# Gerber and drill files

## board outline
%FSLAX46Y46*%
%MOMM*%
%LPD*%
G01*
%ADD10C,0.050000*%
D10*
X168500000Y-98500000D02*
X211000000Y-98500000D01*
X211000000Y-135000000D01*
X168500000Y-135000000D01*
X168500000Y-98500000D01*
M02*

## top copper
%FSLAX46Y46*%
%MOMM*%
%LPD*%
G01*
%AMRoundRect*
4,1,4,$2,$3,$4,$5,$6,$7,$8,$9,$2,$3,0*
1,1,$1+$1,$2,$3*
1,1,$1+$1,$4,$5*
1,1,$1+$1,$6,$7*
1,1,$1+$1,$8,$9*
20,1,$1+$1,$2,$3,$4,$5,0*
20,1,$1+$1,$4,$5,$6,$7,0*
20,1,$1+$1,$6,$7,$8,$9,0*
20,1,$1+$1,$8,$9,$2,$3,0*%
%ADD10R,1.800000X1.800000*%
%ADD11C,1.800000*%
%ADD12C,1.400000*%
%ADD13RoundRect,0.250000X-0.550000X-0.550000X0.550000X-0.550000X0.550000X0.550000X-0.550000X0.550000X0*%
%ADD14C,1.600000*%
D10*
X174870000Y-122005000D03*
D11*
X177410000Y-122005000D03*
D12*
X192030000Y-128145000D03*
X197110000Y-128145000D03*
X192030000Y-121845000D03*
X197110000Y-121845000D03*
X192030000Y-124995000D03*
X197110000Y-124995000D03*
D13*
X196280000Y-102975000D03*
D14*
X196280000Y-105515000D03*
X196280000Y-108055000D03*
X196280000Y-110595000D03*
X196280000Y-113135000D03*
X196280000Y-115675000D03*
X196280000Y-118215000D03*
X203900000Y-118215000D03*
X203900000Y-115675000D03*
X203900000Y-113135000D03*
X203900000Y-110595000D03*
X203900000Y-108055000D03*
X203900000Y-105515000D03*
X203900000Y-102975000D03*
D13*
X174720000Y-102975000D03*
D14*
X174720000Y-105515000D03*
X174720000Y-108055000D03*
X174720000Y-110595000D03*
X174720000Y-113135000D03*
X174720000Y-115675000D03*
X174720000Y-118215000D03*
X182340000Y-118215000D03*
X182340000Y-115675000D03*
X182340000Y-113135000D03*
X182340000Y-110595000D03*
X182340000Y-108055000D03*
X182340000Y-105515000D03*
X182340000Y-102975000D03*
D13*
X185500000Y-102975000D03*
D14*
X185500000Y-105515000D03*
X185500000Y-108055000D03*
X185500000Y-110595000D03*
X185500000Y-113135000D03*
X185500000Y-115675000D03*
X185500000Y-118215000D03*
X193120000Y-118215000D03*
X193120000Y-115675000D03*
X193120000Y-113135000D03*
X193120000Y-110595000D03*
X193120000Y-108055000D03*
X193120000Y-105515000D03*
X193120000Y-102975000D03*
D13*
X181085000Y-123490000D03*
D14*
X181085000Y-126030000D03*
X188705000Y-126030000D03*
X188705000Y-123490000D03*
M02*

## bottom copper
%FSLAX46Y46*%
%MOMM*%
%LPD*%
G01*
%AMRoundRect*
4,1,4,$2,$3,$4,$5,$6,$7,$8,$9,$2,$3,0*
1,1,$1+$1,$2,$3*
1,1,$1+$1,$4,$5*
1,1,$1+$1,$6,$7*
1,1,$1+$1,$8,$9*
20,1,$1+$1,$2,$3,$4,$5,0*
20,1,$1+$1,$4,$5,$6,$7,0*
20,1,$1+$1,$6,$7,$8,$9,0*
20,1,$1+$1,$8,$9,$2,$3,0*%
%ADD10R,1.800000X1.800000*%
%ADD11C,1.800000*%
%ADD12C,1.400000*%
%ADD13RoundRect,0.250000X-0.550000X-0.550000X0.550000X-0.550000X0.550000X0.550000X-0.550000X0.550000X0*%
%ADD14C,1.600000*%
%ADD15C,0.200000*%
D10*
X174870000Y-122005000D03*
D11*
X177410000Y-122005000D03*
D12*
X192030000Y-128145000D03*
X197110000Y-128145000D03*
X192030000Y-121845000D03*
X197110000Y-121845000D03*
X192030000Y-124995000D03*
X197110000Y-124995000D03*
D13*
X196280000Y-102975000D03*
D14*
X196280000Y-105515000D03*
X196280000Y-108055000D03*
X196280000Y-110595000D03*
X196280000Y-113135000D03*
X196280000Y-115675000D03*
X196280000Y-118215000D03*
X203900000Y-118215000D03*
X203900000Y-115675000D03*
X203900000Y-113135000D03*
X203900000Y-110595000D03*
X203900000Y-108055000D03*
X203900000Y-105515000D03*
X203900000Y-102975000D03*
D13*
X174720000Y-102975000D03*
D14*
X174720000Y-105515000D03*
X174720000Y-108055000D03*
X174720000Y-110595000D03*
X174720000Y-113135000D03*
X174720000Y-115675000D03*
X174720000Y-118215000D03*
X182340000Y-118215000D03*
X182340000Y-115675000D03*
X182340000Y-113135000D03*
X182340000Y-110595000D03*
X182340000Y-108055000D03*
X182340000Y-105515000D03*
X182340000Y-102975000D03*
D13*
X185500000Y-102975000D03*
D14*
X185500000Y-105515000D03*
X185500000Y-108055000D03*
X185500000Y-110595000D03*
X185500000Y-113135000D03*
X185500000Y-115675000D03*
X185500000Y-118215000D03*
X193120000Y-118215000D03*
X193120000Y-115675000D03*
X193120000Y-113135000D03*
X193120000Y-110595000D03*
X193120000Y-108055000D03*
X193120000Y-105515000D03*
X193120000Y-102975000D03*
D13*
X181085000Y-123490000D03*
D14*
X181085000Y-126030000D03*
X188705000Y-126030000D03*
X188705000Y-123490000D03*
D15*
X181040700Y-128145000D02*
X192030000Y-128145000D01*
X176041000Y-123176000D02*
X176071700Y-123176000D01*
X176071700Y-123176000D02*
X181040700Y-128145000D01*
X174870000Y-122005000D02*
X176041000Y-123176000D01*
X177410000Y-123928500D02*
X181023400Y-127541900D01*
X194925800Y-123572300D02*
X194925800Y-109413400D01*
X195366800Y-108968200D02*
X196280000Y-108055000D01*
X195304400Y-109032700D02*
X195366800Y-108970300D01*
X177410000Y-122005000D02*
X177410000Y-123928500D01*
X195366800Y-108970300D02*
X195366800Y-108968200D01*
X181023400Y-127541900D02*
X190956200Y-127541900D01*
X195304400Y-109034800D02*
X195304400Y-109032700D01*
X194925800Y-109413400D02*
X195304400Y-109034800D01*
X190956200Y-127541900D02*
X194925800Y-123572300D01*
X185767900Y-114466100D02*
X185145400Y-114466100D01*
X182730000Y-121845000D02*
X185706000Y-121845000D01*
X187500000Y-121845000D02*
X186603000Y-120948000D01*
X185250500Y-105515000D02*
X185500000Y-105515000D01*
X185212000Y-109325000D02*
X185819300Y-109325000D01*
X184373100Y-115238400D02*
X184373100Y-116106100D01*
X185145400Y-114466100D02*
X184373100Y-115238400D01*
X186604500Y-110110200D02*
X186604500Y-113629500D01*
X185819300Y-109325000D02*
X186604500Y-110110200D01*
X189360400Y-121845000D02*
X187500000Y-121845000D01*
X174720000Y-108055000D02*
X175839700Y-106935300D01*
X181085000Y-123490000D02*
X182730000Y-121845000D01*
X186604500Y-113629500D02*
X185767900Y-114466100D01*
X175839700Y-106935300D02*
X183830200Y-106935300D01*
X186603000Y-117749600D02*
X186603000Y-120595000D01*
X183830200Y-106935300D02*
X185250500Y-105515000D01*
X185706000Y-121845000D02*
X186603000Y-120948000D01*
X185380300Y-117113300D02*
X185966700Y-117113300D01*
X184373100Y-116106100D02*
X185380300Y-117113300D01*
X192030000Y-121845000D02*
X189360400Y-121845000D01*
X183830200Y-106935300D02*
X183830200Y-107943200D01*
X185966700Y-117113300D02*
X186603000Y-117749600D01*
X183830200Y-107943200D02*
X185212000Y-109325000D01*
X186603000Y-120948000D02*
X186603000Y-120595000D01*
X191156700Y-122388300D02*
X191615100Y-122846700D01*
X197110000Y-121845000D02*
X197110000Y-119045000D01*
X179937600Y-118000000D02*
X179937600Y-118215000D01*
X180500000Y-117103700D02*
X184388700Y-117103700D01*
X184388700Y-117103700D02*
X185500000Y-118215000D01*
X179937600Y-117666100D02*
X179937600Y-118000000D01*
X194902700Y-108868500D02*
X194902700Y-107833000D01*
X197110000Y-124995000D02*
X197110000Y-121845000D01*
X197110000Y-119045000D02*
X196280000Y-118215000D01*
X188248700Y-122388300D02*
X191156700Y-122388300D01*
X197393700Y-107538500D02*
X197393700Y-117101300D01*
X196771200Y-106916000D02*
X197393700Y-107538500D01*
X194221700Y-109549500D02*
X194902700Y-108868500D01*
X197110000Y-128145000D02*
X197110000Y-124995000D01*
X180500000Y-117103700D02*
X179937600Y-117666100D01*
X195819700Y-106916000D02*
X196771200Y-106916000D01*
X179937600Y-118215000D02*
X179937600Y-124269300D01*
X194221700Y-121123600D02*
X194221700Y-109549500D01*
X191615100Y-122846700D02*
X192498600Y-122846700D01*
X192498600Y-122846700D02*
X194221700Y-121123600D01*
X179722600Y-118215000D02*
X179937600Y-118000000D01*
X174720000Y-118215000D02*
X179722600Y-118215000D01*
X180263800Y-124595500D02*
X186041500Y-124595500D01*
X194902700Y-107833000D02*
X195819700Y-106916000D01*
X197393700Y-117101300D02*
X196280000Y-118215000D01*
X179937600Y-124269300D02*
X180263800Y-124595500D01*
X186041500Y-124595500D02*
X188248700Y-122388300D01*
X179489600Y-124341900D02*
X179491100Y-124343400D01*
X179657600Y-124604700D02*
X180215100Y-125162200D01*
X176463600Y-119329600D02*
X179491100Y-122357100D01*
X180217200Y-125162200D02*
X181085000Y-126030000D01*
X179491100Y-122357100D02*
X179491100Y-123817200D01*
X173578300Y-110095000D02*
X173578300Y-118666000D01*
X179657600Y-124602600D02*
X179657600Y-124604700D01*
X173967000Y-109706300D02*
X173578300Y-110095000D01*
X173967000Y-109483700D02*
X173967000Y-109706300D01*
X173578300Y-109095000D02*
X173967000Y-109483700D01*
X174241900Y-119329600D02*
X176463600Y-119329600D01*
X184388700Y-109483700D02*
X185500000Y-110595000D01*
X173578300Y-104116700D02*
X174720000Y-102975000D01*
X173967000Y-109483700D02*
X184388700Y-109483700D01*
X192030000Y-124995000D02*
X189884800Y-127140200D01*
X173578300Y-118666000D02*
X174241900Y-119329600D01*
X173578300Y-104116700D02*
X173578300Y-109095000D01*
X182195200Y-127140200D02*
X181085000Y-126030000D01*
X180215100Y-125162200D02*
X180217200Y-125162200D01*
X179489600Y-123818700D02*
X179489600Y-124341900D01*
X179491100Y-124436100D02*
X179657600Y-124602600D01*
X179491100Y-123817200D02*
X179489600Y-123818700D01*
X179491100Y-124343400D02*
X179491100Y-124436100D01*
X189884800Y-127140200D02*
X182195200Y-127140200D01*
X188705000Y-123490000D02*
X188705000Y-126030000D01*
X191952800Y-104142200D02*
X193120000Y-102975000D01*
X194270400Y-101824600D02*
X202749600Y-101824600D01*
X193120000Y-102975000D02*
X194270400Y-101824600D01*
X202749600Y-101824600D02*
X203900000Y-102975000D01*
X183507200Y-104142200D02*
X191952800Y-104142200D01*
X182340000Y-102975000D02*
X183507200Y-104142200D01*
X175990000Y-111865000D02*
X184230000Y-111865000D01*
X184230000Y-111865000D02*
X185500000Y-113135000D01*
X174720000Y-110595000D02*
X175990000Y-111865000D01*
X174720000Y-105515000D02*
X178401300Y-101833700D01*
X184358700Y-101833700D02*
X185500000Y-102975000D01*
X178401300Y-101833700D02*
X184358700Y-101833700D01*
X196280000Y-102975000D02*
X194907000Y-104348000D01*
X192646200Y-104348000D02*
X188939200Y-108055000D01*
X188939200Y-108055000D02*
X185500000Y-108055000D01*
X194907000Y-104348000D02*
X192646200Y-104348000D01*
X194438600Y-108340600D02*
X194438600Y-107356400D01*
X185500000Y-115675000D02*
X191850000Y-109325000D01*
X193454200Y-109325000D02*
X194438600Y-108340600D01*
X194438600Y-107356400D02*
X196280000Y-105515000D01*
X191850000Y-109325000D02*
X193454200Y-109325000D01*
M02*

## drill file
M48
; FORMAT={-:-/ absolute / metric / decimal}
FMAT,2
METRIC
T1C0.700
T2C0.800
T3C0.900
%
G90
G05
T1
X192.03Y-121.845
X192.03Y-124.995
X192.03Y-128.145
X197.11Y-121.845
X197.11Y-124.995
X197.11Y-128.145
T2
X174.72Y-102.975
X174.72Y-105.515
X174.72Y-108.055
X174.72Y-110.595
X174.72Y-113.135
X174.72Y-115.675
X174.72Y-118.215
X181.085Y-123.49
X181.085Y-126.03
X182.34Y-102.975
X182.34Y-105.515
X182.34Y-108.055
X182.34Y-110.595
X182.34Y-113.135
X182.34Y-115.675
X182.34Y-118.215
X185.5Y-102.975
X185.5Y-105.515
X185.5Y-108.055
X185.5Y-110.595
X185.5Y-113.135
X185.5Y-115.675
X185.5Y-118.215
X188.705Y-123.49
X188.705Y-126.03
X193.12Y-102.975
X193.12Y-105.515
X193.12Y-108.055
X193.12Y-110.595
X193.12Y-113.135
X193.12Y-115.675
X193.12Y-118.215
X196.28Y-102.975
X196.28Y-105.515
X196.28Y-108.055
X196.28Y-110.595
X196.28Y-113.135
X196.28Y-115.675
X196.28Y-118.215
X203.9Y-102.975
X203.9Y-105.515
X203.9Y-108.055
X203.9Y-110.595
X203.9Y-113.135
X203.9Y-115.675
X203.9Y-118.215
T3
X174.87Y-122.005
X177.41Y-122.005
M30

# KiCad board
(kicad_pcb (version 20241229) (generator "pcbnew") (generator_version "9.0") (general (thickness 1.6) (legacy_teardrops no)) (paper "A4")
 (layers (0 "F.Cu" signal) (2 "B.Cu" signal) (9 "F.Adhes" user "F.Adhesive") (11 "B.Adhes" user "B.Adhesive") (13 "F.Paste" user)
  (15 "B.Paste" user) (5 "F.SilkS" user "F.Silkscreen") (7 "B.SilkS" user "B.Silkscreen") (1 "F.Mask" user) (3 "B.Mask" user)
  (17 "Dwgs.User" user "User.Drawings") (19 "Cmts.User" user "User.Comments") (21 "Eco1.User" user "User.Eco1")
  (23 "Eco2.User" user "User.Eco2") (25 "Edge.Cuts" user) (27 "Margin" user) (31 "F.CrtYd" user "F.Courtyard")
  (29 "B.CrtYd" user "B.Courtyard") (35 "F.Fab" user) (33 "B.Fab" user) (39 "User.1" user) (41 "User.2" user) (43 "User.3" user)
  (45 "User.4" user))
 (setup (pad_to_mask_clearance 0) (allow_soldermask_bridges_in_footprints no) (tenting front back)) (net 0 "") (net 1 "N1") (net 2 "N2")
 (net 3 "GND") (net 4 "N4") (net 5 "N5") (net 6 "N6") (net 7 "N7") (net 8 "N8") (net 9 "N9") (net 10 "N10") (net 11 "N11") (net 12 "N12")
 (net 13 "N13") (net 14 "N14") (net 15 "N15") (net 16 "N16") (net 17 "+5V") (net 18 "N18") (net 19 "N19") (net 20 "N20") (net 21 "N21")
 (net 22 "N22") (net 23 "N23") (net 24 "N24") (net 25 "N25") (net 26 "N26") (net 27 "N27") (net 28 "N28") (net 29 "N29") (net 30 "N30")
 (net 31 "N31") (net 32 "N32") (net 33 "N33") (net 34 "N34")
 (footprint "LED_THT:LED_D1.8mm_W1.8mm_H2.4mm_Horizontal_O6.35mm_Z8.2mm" (layer "F.Cu") (at 174.87 122.005)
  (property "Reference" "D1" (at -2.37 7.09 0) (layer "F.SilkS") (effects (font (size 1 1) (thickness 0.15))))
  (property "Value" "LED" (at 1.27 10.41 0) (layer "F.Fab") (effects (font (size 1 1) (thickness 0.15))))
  (pad "1" thru_hole rect (at 0 0) (size 1.8 1.8) (drill 0.9) (layers "*.Cu" "*.Mask") (remove_unused_layers no) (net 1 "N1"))
  (pad "2" thru_hole circle (at 2.54 0) (size 1.8 1.8) (drill 0.9) (layers "*.Cu" "*.Mask") (remove_unused_layers no) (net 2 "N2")))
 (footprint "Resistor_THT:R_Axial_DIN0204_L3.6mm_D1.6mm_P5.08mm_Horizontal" (layer "F.Cu") (at 192.03 128.145)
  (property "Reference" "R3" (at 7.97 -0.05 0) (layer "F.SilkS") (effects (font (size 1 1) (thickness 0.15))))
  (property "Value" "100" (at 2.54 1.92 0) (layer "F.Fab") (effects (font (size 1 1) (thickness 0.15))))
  (pad "1" thru_hole circle (at 0 0) (size 1.4 1.4) (drill 0.7) (layers "*.Cu" "*.Mask") (remove_unused_layers no) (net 1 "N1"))
  (pad "2" thru_hole circle (at 5.08 0) (size 1.4 1.4) (drill 0.7) (layers "*.Cu" "*.Mask") (remove_unused_layers no) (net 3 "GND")))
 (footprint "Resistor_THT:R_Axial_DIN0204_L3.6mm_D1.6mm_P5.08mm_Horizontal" (layer "F.Cu") (at 192.03 121.845)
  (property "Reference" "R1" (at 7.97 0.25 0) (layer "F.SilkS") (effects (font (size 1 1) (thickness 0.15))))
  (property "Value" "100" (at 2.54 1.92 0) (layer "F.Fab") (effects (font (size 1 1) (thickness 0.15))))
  (pad "1" thru_hole circle (at 0 0) (size 1.4 1.4) (drill 0.7) (layers "*.Cu" "*.Mask") (remove_unused_layers no) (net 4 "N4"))
  (pad "2" thru_hole circle (at 5.08 0) (size 1.4 1.4) (drill 0.7) (layers "*.Cu" "*.Mask") (remove_unused_layers no) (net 3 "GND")))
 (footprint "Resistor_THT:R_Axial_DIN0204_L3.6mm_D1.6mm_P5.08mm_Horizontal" (layer "F.Cu") (at 192.03 124.995)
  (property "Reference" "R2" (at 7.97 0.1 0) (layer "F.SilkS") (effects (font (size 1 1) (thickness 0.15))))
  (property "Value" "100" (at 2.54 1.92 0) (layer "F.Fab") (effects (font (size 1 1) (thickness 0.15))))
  (pad "1" thru_hole circle (at 0 0) (size 1.4 1.4) (drill 0.7) (layers "*.Cu" "*.Mask") (remove_unused_layers no) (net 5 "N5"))
  (pad "2" thru_hole circle (at 5.08 0) (size 1.4 1.4) (drill 0.7) (layers "*.Cu" "*.Mask") (remove_unused_layers no) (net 3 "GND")))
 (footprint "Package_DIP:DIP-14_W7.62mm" (layer "F.Cu") (at 196.28 102.975)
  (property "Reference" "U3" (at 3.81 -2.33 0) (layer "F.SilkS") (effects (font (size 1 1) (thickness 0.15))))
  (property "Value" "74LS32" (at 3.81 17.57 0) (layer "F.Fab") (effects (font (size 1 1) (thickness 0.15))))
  (pad "1" thru_hole roundrect (at 0 0) (size 1.6 1.6) (drill 0.8) (layers "*.Cu" "*.Mask") (remove_unused_layers no)
   (roundrect_rratio 0.15625) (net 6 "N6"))
  (pad "2" thru_hole circle (at 0 2.54) (size 1.6 1.6) (drill 0.8) (layers "*.Cu" "*.Mask") (remove_unused_layers no) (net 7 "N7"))
  (pad "3" thru_hole circle (at 0 5.08) (size 1.6 1.6) (drill 0.8) (layers "*.Cu" "*.Mask") (remove_unused_layers no) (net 2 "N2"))
  (pad "4" thru_hole circle (at 0 7.62) (size 1.6 1.6) (drill 0.8) (layers "*.Cu" "*.Mask") (remove_unused_layers no) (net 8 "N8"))
  (pad "5" thru_hole circle (at 0 10.16) (size 1.6 1.6) (drill 0.8) (layers "*.Cu" "*.Mask") (remove_unused_layers no) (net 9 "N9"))
  (pad "6" thru_hole circle (at 0 12.7) (size 1.6 1.6) (drill 0.8) (layers "*.Cu" "*.Mask") (remove_unused_layers no) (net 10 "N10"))
  (pad "7" thru_hole circle (at 0 15.24) (size 1.6 1.6) (drill 0.8) (layers "*.Cu" "*.Mask") (remove_unused_layers no) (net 3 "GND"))
  (pad "8" thru_hole circle (at 7.62 15.24) (size 1.6 1.6) (drill 0.8) (layers "*.Cu" "*.Mask") (remove_unused_layers no) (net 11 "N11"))
  (pad "9" thru_hole circle (at 7.62 12.7) (size 1.6 1.6) (drill 0.8) (layers "*.Cu" "*.Mask") (remove_unused_layers no) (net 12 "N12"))
  (pad "10" thru_hole circle (at 7.62 10.16) (size 1.6 1.6) (drill 0.8) (layers "*.Cu" "*.Mask") (remove_unused_layers no) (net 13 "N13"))
  (pad "11" thru_hole circle (at 7.62 7.62) (size 1.6 1.6) (drill 0.8) (layers "*.Cu" "*.Mask") (remove_unused_layers no) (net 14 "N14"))
  (pad "12" thru_hole circle (at 7.62 5.08) (size 1.6 1.6) (drill 0.8) (layers "*.Cu" "*.Mask") (remove_unused_layers no) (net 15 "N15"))
  (pad "13" thru_hole circle (at 7.62 2.54) (size 1.6 1.6) (drill 0.8) (layers "*.Cu" "*.Mask") (remove_unused_layers no) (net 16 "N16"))
  (pad "14" thru_hole circle (at 7.62 0) (size 1.6 1.6) (drill 0.8) (layers "*.Cu" "*.Mask") (remove_unused_layers no) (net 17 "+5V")))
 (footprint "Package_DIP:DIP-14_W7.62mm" (layer "F.Cu") (at 174.72 102.975)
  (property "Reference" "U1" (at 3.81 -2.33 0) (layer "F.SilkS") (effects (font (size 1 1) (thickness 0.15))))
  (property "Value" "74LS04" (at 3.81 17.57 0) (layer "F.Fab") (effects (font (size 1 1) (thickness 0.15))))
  (pad "1" thru_hole roundrect (at 0 0) (size 1.6 1.6) (drill 0.8) (layers "*.Cu" "*.Mask") (remove_unused_layers no)
   (roundrect_rratio 0.15625) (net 5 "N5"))
  (pad "2" thru_hole circle (at 0 2.54) (size 1.6 1.6) (drill 0.8) (layers "*.Cu" "*.Mask") (remove_unused_layers no) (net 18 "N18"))
  (pad "3" thru_hole circle (at 0 5.08) (size 1.6 1.6) (drill 0.8) (layers "*.Cu" "*.Mask") (remove_unused_layers no) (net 4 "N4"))
  (pad "4" thru_hole circle (at 0 7.62) (size 1.6 1.6) (drill 0.8) (layers "*.Cu" "*.Mask") (remove_unused_layers no) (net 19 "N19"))
  (pad "5" thru_hole circle (at 0 10.16) (size 1.6 1.6) (drill 0.8) (layers "*.Cu" "*.Mask") (remove_unused_layers no) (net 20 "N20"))
  (pad "6" thru_hole circle (at 0 12.7) (size 1.6 1.6) (drill 0.8) (layers "*.Cu" "*.Mask") (remove_unused_layers no) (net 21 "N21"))
  (pad "7" thru_hole circle (at 0 15.24) (size 1.6 1.6) (drill 0.8) (layers "*.Cu" "*.Mask") (remove_unused_layers no) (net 3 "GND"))
  (pad "8" thru_hole circle (at 7.62 15.24) (size 1.6 1.6) (drill 0.8) (layers "*.Cu" "*.Mask") (remove_unused_layers no) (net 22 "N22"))
  (pad "9" thru_hole circle (at 7.62 12.7) (size 1.6 1.6) (drill 0.8) (layers "*.Cu" "*.Mask") (remove_unused_layers no) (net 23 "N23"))
  (pad "10" thru_hole circle (at 7.62 10.16) (size 1.6 1.6) (drill 0.8) (layers "*.Cu" "*.Mask") (remove_unused_layers no) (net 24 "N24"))
  (pad "11" thru_hole circle (at 7.62 7.62) (size 1.6 1.6) (drill 0.8) (layers "*.Cu" "*.Mask") (remove_unused_layers no) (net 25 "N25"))
  (pad "12" thru_hole circle (at 7.62 5.08) (size 1.6 1.6) (drill 0.8) (layers "*.Cu" "*.Mask") (remove_unused_layers no) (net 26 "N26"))
  (pad "13" thru_hole circle (at 7.62 2.54) (size 1.6 1.6) (drill 0.8) (layers "*.Cu" "*.Mask") (remove_unused_layers no) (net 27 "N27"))
  (pad "14" thru_hole circle (at 7.62 0) (size 1.6 1.6) (drill 0.8) (layers "*.Cu" "*.Mask") (remove_unused_layers no) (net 17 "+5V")))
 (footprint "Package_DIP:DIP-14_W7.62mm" (layer "F.Cu") (at 185.5 102.975)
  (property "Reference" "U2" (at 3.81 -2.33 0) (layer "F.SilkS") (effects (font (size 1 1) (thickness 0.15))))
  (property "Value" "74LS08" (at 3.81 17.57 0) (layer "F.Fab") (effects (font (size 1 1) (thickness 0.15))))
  (pad "1" thru_hole roundrect (at 0 0) (size 1.6 1.6) (drill 0.8) (layers "*.Cu" "*.Mask") (remove_unused_layers no)
   (roundrect_rratio 0.15625) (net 18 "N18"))
  (pad "2" thru_hole circle (at 0 2.54) (size 1.6 1.6) (drill 0.8) (layers "*.Cu" "*.Mask") (remove_unused_layers no) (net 4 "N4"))
  (pad "3" thru_hole circle (at 0 5.08) (size 1.6 1.6) (drill 0.8) (layers "*.Cu" "*.Mask") (remove_unused_layers no) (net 6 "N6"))
  (pad "4" thru_hole circle (at 0 7.62) (size 1.6 1.6) (drill 0.8) (layers "*.Cu" "*.Mask") (remove_unused_layers no) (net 5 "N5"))
  (pad "5" thru_hole circle (at 0 10.16) (size 1.6 1.6) (drill 0.8) (layers "*.Cu" "*.Mask") (remove_unused_layers no) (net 19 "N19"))
  (pad "6" thru_hole circle (at 0 12.7) (size 1.6 1.6) (drill 0.8) (layers "*.Cu" "*.Mask") (remove_unused_layers no) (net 7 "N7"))
  (pad "7" thru_hole circle (at 0 15.24) (size 1.6 1.6) (drill 0.8) (layers "*.Cu" "*.Mask") (remove_unused_layers no) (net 3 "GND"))
  (pad "8" thru_hole circle (at 7.62 15.24) (size 1.6 1.6) (drill 0.8) (layers "*.Cu" "*.Mask") (remove_unused_layers no) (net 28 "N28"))
  (pad "9" thru_hole circle (at 7.62 12.7) (size 1.6 1.6) (drill 0.8) (layers "*.Cu" "*.Mask") (remove_unused_layers no) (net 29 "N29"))
  (pad "10" thru_hole circle (at 7.62 10.16) (size 1.6 1.6) (drill 0.8) (layers "*.Cu" "*.Mask") (remove_unused_layers no) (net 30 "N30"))
  (pad "11" thru_hole circle (at 7.62 7.62) (size 1.6 1.6) (drill 0.8) (layers "*.Cu" "*.Mask") (remove_unused_layers no) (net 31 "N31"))
  (pad "12" thru_hole circle (at 7.62 5.08) (size 1.6 1.6) (drill 0.8) (layers "*.Cu" "*.Mask") (remove_unused_layers no) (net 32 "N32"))
  (pad "13" thru_hole circle (at 7.62 2.54) (size 1.6 1.6) (drill 0.8) (layers "*.Cu" "*.Mask") (remove_unused_layers no) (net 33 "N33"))
  (pad "14" thru_hole circle (at 7.62 0) (size 1.6 1.6) (drill 0.8) (layers "*.Cu" "*.Mask") (remove_unused_layers no) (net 17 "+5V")))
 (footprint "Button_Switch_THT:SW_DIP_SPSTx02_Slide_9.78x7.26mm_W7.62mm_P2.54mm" (layer "F.Cu") (at 181.085 123.49)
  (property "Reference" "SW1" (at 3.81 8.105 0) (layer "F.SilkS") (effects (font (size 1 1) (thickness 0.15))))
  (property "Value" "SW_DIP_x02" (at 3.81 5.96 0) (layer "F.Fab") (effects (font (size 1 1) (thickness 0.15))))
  (pad "1" thru_hole roundrect (at 0 0) (size 1.6 1.6) (drill 0.8) (layers "*.Cu" "*.Mask") (remove_unused_layers no)
   (roundrect_rratio 0.15625) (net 4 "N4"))
  (pad "2" thru_hole circle (at 0 2.54) (size 1.6 1.6) (drill 0.8) (layers "*.Cu" "*.Mask") (remove_unused_layers no) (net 5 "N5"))
  (pad "3" thru_hole circle (at 7.62 2.54) (size 1.6 1.6) (drill 0.8) (layers "*.Cu" "*.Mask") (remove_unused_layers no) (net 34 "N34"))
  (pad "4" thru_hole circle (at 7.62 0) (size 1.6 1.6) (drill 0.8) (layers "*.Cu" "*.Mask") (remove_unused_layers no) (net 34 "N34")))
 (gr_rect (start 168.5 98.5) (end 211 135) (stroke (width 0.05) (type default)) (fill no) (layer "Edge.Cuts"))
 (segment (start 181.0407 128.145) (end 192.03 128.145) (width 0.2) (layer "B.Cu") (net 1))
 (segment (start 176.041 123.176) (end 176.0717 123.176) (width 0.2) (layer "B.Cu") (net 1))
 (segment (start 176.0717 123.176) (end 181.0407 128.145) (width 0.2) (layer "B.Cu") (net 1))
 (segment (start 174.87 122.005) (end 176.041 123.176) (width 0.2) (layer "B.Cu") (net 1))
 (segment (start 177.41 123.9285) (end 181.0234 127.5419) (width 0.2) (layer "B.Cu") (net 2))
 (segment (start 194.9258 123.5723) (end 194.9258 109.4134) (width 0.2) (layer "B.Cu") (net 2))
 (segment (start 195.3668 108.9682) (end 196.28 108.055) (width 0.2) (layer "B.Cu") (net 2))
 (segment (start 195.3044 109.0327) (end 195.3668 108.9703) (width 0.2) (layer "B.Cu") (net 2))
 (segment (start 177.41 122.005) (end 177.41 123.9285) (width 0.2) (layer "B.Cu") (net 2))
 (segment (start 195.3668 108.9703) (end 195.3668 108.9682) (width 0.2) (layer "B.Cu") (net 2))
 (segment (start 181.0234 127.5419) (end 190.9562 127.5419) (width 0.2) (layer "B.Cu") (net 2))
 (segment (start 195.3044 109.0348) (end 195.3044 109.0327) (width 0.2) (layer "B.Cu") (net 2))
 (segment (start 194.9258 109.4134) (end 195.3044 109.0348) (width 0.2) (layer "B.Cu") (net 2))
 (segment (start 190.9562 127.5419) (end 194.9258 123.5723) (width 0.2) (layer "B.Cu") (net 2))
 (segment (start 185.7679 114.4661) (end 185.1454 114.4661) (width 0.2) (layer "B.Cu") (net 4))
 (segment (start 182.73 121.845) (end 185.706 121.845) (width 0.2) (layer "B.Cu") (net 4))
 (segment (start 187.5 121.845) (end 186.603 120.948) (width 0.2) (layer "B.Cu") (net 4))
 (segment (start 185.2505 105.515) (end 185.5 105.515) (width 0.2) (layer "B.Cu") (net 4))
 (segment (start 185.212 109.325) (end 185.8193 109.325) (width 0.2) (layer "B.Cu") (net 4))
 (segment (start 184.3731 115.2384) (end 184.3731 116.1061) (width 0.2) (layer "B.Cu") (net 4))
 (segment (start 185.1454 114.4661) (end 184.3731 115.2384) (width 0.2) (layer "B.Cu") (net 4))
 (segment (start 186.6045 110.1102) (end 186.6045 113.6295) (width 0.2) (layer "B.Cu") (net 4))
 (segment (start 185.8193 109.325) (end 186.6045 110.1102) (width 0.2) (layer "B.Cu") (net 4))
 (segment (start 189.3604 121.845) (end 187.5 121.845) (width 0.2) (layer "B.Cu") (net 4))
 (segment (start 174.72 108.055) (end 175.8397 106.9353) (width 0.2) (layer "B.Cu") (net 4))
 (segment (start 181.085 123.49) (end 182.73 121.845) (width 0.2) (layer "B.Cu") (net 4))
 (segment (start 186.6045 113.6295) (end 185.7679 114.4661) (width 0.2) (layer "B.Cu") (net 4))
 (segment (start 175.8397 106.9353) (end 183.8302 106.9353) (width 0.2) (layer "B.Cu") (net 4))
 (segment (start 186.603 117.7496) (end 186.603 120.595) (width 0.2) (layer "B.Cu") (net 4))
 (segment (start 183.8302 106.9353) (end 185.2505 105.515) (width 0.2) (layer "B.Cu") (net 4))
 (segment (start 185.706 121.845) (end 186.603 120.948) (width 0.2) (layer "B.Cu") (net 4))
 (segment (start 185.3803 117.1133) (end 185.9667 117.1133) (width 0.2) (layer "B.Cu") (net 4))
 (segment (start 184.3731 116.1061) (end 185.3803 117.1133) (width 0.2) (layer "B.Cu") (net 4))
 (segment (start 192.03 121.845) (end 189.3604 121.845) (width 0.2) (layer "B.Cu") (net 4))
 (segment (start 183.8302 106.9353) (end 183.8302 107.9432) (width 0.2) (layer "B.Cu") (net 4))
 (segment (start 185.9667 117.1133) (end 186.603 117.7496) (width 0.2) (layer "B.Cu") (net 4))
 (segment (start 183.8302 107.9432) (end 185.212 109.325) (width 0.2) (layer "B.Cu") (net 4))
 (segment (start 186.603 120.948) (end 186.603 120.595) (width 0.2) (layer "B.Cu") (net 4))
 (segment (start 191.1567 122.3883) (end 191.6151 122.8467) (width 0.2) (layer "B.Cu") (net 3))
 (segment (start 197.11 121.845) (end 197.11 119.045) (width 0.2) (layer "B.Cu") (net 3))
 (segment (start 179.9376 118) (end 179.9376 118.215) (width 0.2) (layer "B.Cu") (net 3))
 (segment (start 180.5 117.1037) (end 184.3887 117.1037) (width 0.2) (layer "B.Cu") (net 3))
 (segment (start 184.3887 117.1037) (end 185.5 118.215) (width 0.2) (layer "B.Cu") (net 3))
 (segment (start 179.9376 117.6661) (end 179.9376 118) (width 0.2) (layer "B.Cu") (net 3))
 (segment (start 194.9027 108.8685) (end 194.9027 107.833) (width 0.2) (layer "B.Cu") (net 3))
 (segment (start 197.11 124.995) (end 197.11 121.845) (width 0.2) (layer "B.Cu") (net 3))
 (segment (start 197.11 119.045) (end 196.28 118.215) (width 0.2) (layer "B.Cu") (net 3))
 (segment (start 188.2487 122.3883) (end 191.1567 122.3883) (width 0.2) (layer "B.Cu") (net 3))
 (segment (start 197.3937 107.5385) (end 197.3937 117.1013) (width 0.2) (layer "B.Cu") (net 3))
 (segment (start 196.7712 106.916) (end 197.3937 107.5385) (width 0.2) (layer "B.Cu") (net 3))
 (segment (start 194.2217 109.5495) (end 194.9027 108.8685) (width 0.2) (layer "B.Cu") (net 3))
 (segment (start 197.11 128.145) (end 197.11 124.995) (width 0.2) (layer "B.Cu") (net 3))
 (segment (start 180.5 117.1037) (end 179.9376 117.6661) (width 0.2) (layer "B.Cu") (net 3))
 (segment (start 195.8197 106.916) (end 196.7712 106.916) (width 0.2) (layer "B.Cu") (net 3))
 (segment (start 179.9376 118.215) (end 179.9376 124.2693) (width 0.2) (layer "B.Cu") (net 3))
 (segment (start 194.2217 121.1236) (end 194.2217 109.5495) (width 0.2) (layer "B.Cu") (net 3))
 (segment (start 191.6151 122.8467) (end 192.4986 122.8467) (width 0.2) (layer "B.Cu") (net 3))
 (segment (start 192.4986 122.8467) (end 194.2217 121.1236) (width 0.2) (layer "B.Cu") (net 3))
 (segment (start 179.7226 118.215) (end 179.9376 118) (width 0.2) (layer "B.Cu") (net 3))
 (segment (start 174.72 118.215) (end 179.7226 118.215) (width 0.2) (layer "B.Cu") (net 3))
 (segment (start 180.2638 124.5955) (end 186.0415 124.5955) (width 0.2) (layer "B.Cu") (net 3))
 (segment (start 194.9027 107.833) (end 195.8197 106.916) (width 0.2) (layer "B.Cu") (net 3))
 (segment (start 197.3937 117.1013) (end 196.28 118.215) (width 0.2) (layer "B.Cu") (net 3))
 (segment (start 179.9376 124.2693) (end 180.2638 124.5955) (width 0.2) (layer "B.Cu") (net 3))
 (segment (start 186.0415 124.5955) (end 188.2487 122.3883) (width 0.2) (layer "B.Cu") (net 3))
 (segment (start 179.4896 124.3419) (end 179.4911 124.3434) (width 0.2) (layer "B.Cu") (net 5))
 (segment (start 179.6576 124.6047) (end 180.2151 125.1622) (width 0.2) (layer "B.Cu") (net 5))
 (segment (start 176.4636 119.3296) (end 179.4911 122.3571) (width 0.2) (layer "B.Cu") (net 5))
 (segment (start 180.2172 125.1622) (end 181.085 126.03) (width 0.2) (layer "B.Cu") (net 5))
 (segment (start 179.4911 122.3571) (end 179.4911 123.8172) (width 0.2) (layer "B.Cu") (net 5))
 (segment (start 173.5783 110.095) (end 173.5783 118.666) (width 0.2) (layer "B.Cu") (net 5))
 (segment (start 179.6576 124.6026) (end 179.6576 124.6047) (width 0.2) (layer "B.Cu") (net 5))
 (segment (start 173.967 109.7063) (end 173.5783 110.095) (width 0.2) (layer "B.Cu") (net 5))
 (segment (start 173.967 109.4837) (end 173.967 109.7063) (width 0.2) (layer "B.Cu") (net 5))
 (segment (start 173.5783 109.095) (end 173.967 109.4837) (width 0.2) (layer "B.Cu") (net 5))
 (segment (start 174.2419 119.3296) (end 176.4636 119.3296) (width 0.2) (layer "B.Cu") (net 5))
 (segment (start 184.3887 109.4837) (end 185.5 110.595) (width 0.2) (layer "B.Cu") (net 5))
 (segment (start 173.5783 104.1167) (end 174.72 102.975) (width 0.2) (layer "B.Cu") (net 5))
 (segment (start 173.967 109.4837) (end 184.3887 109.4837) (width 0.2) (layer "B.Cu") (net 5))
 (segment (start 192.03 124.995) (end 189.8848 127.1402) (width 0.2) (layer "B.Cu") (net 5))
 (segment (start 173.5783 118.666) (end 174.2419 119.3296) (width 0.2) (layer "B.Cu") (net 5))
 (segment (start 173.5783 104.1167) (end 173.5783 109.095) (width 0.2) (layer "B.Cu") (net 5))
 (segment (start 182.1952 127.1402) (end 181.085 126.03) (width 0.2) (layer "B.Cu") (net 5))
 (segment (start 180.2151 125.1622) (end 180.2172 125.1622) (width 0.2) (layer "B.Cu") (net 5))
 (segment (start 179.4896 123.8187) (end 179.4896 124.3419) (width 0.2) (layer "B.Cu") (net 5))
 (segment (start 179.4911 124.4361) (end 179.6576 124.6026) (width 0.2) (layer "B.Cu") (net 5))
 (segment (start 179.4911 123.8172) (end 179.4896 123.8187) (width 0.2) (layer "B.Cu") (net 5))
 (segment (start 179.4911 124.3434) (end 179.4911 124.4361) (width 0.2) (layer "B.Cu") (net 5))
 (segment (start 189.8848 127.1402) (end 182.1952 127.1402) (width 0.2) (layer "B.Cu") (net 5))
 (segment (start 188.705 123.49) (end 188.705 126.03) (width 0.2) (layer "B.Cu") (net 34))
 (segment (start 191.9528 104.1422) (end 193.12 102.975) (width 0.2) (layer "B.Cu") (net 17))
 (segment (start 194.2704 101.8246) (end 202.7496 101.8246) (width 0.2) (layer "B.Cu") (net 17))
 (segment (start 193.12 102.975) (end 194.2704 101.8246) (width 0.2) (layer "B.Cu") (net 17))
 (segment (start 202.7496 101.8246) (end 203.9 102.975) (width 0.2) (layer "B.Cu") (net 17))
 (segment (start 183.5072 104.1422) (end 191.9528 104.1422) (width 0.2) (layer "B.Cu") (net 17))
 (segment (start 182.34 102.975) (end 183.5072 104.1422) (width 0.2) (layer "B.Cu") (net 17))
 (segment (start 175.99 111.865) (end 184.23 111.865) (width 0.2) (layer "B.Cu") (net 19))
 (segment (start 184.23 111.865) (end 185.5 113.135) (width 0.2) (layer "B.Cu") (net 19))
 (segment (start 174.72 110.595) (end 175.99 111.865) (width 0.2) (layer "B.Cu") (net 19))
 (segment (start 174.72 105.515) (end 178.4013 101.8337) (width 0.2) (layer "B.Cu") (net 18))
 (segment (start 184.3587 101.8337) (end 185.5 102.975) (width 0.2) (layer "B.Cu") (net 18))
 (segment (start 178.4013 101.8337) (end 184.3587 101.8337) (width 0.2) (layer "B.Cu") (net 18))
 (segment (start 196.28 102.975) (end 194.907 104.348) (width 0.2) (layer "B.Cu") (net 6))
 (segment (start 192.6462 104.348) (end 188.9392 108.055) (width 0.2) (layer "B.Cu") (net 6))
 (segment (start 188.9392 108.055) (end 185.5 108.055) (width 0.2) (layer "B.Cu") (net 6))
 (segment (start 194.907 104.348) (end 192.6462 104.348) (width 0.2) (layer "B.Cu") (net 6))
 (segment (start 194.4386 108.3406) (end 194.4386 107.3564) (width 0.2) (layer "B.Cu") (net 7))
 (segment (start 185.5 115.675) (end 191.85 109.325) (width 0.2) (layer "B.Cu") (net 7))
 (segment (start 193.4542 109.325) (end 194.4386 108.3406) (width 0.2) (layer "B.Cu") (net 7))
 (segment (start 194.4386 107.3564) (end 196.28 105.515) (width 0.2) (layer "B.Cu") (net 7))
 (segment (start 191.85 109.325) (end 193.4542 109.325) (width 0.2) (layer "B.Cu") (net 7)))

